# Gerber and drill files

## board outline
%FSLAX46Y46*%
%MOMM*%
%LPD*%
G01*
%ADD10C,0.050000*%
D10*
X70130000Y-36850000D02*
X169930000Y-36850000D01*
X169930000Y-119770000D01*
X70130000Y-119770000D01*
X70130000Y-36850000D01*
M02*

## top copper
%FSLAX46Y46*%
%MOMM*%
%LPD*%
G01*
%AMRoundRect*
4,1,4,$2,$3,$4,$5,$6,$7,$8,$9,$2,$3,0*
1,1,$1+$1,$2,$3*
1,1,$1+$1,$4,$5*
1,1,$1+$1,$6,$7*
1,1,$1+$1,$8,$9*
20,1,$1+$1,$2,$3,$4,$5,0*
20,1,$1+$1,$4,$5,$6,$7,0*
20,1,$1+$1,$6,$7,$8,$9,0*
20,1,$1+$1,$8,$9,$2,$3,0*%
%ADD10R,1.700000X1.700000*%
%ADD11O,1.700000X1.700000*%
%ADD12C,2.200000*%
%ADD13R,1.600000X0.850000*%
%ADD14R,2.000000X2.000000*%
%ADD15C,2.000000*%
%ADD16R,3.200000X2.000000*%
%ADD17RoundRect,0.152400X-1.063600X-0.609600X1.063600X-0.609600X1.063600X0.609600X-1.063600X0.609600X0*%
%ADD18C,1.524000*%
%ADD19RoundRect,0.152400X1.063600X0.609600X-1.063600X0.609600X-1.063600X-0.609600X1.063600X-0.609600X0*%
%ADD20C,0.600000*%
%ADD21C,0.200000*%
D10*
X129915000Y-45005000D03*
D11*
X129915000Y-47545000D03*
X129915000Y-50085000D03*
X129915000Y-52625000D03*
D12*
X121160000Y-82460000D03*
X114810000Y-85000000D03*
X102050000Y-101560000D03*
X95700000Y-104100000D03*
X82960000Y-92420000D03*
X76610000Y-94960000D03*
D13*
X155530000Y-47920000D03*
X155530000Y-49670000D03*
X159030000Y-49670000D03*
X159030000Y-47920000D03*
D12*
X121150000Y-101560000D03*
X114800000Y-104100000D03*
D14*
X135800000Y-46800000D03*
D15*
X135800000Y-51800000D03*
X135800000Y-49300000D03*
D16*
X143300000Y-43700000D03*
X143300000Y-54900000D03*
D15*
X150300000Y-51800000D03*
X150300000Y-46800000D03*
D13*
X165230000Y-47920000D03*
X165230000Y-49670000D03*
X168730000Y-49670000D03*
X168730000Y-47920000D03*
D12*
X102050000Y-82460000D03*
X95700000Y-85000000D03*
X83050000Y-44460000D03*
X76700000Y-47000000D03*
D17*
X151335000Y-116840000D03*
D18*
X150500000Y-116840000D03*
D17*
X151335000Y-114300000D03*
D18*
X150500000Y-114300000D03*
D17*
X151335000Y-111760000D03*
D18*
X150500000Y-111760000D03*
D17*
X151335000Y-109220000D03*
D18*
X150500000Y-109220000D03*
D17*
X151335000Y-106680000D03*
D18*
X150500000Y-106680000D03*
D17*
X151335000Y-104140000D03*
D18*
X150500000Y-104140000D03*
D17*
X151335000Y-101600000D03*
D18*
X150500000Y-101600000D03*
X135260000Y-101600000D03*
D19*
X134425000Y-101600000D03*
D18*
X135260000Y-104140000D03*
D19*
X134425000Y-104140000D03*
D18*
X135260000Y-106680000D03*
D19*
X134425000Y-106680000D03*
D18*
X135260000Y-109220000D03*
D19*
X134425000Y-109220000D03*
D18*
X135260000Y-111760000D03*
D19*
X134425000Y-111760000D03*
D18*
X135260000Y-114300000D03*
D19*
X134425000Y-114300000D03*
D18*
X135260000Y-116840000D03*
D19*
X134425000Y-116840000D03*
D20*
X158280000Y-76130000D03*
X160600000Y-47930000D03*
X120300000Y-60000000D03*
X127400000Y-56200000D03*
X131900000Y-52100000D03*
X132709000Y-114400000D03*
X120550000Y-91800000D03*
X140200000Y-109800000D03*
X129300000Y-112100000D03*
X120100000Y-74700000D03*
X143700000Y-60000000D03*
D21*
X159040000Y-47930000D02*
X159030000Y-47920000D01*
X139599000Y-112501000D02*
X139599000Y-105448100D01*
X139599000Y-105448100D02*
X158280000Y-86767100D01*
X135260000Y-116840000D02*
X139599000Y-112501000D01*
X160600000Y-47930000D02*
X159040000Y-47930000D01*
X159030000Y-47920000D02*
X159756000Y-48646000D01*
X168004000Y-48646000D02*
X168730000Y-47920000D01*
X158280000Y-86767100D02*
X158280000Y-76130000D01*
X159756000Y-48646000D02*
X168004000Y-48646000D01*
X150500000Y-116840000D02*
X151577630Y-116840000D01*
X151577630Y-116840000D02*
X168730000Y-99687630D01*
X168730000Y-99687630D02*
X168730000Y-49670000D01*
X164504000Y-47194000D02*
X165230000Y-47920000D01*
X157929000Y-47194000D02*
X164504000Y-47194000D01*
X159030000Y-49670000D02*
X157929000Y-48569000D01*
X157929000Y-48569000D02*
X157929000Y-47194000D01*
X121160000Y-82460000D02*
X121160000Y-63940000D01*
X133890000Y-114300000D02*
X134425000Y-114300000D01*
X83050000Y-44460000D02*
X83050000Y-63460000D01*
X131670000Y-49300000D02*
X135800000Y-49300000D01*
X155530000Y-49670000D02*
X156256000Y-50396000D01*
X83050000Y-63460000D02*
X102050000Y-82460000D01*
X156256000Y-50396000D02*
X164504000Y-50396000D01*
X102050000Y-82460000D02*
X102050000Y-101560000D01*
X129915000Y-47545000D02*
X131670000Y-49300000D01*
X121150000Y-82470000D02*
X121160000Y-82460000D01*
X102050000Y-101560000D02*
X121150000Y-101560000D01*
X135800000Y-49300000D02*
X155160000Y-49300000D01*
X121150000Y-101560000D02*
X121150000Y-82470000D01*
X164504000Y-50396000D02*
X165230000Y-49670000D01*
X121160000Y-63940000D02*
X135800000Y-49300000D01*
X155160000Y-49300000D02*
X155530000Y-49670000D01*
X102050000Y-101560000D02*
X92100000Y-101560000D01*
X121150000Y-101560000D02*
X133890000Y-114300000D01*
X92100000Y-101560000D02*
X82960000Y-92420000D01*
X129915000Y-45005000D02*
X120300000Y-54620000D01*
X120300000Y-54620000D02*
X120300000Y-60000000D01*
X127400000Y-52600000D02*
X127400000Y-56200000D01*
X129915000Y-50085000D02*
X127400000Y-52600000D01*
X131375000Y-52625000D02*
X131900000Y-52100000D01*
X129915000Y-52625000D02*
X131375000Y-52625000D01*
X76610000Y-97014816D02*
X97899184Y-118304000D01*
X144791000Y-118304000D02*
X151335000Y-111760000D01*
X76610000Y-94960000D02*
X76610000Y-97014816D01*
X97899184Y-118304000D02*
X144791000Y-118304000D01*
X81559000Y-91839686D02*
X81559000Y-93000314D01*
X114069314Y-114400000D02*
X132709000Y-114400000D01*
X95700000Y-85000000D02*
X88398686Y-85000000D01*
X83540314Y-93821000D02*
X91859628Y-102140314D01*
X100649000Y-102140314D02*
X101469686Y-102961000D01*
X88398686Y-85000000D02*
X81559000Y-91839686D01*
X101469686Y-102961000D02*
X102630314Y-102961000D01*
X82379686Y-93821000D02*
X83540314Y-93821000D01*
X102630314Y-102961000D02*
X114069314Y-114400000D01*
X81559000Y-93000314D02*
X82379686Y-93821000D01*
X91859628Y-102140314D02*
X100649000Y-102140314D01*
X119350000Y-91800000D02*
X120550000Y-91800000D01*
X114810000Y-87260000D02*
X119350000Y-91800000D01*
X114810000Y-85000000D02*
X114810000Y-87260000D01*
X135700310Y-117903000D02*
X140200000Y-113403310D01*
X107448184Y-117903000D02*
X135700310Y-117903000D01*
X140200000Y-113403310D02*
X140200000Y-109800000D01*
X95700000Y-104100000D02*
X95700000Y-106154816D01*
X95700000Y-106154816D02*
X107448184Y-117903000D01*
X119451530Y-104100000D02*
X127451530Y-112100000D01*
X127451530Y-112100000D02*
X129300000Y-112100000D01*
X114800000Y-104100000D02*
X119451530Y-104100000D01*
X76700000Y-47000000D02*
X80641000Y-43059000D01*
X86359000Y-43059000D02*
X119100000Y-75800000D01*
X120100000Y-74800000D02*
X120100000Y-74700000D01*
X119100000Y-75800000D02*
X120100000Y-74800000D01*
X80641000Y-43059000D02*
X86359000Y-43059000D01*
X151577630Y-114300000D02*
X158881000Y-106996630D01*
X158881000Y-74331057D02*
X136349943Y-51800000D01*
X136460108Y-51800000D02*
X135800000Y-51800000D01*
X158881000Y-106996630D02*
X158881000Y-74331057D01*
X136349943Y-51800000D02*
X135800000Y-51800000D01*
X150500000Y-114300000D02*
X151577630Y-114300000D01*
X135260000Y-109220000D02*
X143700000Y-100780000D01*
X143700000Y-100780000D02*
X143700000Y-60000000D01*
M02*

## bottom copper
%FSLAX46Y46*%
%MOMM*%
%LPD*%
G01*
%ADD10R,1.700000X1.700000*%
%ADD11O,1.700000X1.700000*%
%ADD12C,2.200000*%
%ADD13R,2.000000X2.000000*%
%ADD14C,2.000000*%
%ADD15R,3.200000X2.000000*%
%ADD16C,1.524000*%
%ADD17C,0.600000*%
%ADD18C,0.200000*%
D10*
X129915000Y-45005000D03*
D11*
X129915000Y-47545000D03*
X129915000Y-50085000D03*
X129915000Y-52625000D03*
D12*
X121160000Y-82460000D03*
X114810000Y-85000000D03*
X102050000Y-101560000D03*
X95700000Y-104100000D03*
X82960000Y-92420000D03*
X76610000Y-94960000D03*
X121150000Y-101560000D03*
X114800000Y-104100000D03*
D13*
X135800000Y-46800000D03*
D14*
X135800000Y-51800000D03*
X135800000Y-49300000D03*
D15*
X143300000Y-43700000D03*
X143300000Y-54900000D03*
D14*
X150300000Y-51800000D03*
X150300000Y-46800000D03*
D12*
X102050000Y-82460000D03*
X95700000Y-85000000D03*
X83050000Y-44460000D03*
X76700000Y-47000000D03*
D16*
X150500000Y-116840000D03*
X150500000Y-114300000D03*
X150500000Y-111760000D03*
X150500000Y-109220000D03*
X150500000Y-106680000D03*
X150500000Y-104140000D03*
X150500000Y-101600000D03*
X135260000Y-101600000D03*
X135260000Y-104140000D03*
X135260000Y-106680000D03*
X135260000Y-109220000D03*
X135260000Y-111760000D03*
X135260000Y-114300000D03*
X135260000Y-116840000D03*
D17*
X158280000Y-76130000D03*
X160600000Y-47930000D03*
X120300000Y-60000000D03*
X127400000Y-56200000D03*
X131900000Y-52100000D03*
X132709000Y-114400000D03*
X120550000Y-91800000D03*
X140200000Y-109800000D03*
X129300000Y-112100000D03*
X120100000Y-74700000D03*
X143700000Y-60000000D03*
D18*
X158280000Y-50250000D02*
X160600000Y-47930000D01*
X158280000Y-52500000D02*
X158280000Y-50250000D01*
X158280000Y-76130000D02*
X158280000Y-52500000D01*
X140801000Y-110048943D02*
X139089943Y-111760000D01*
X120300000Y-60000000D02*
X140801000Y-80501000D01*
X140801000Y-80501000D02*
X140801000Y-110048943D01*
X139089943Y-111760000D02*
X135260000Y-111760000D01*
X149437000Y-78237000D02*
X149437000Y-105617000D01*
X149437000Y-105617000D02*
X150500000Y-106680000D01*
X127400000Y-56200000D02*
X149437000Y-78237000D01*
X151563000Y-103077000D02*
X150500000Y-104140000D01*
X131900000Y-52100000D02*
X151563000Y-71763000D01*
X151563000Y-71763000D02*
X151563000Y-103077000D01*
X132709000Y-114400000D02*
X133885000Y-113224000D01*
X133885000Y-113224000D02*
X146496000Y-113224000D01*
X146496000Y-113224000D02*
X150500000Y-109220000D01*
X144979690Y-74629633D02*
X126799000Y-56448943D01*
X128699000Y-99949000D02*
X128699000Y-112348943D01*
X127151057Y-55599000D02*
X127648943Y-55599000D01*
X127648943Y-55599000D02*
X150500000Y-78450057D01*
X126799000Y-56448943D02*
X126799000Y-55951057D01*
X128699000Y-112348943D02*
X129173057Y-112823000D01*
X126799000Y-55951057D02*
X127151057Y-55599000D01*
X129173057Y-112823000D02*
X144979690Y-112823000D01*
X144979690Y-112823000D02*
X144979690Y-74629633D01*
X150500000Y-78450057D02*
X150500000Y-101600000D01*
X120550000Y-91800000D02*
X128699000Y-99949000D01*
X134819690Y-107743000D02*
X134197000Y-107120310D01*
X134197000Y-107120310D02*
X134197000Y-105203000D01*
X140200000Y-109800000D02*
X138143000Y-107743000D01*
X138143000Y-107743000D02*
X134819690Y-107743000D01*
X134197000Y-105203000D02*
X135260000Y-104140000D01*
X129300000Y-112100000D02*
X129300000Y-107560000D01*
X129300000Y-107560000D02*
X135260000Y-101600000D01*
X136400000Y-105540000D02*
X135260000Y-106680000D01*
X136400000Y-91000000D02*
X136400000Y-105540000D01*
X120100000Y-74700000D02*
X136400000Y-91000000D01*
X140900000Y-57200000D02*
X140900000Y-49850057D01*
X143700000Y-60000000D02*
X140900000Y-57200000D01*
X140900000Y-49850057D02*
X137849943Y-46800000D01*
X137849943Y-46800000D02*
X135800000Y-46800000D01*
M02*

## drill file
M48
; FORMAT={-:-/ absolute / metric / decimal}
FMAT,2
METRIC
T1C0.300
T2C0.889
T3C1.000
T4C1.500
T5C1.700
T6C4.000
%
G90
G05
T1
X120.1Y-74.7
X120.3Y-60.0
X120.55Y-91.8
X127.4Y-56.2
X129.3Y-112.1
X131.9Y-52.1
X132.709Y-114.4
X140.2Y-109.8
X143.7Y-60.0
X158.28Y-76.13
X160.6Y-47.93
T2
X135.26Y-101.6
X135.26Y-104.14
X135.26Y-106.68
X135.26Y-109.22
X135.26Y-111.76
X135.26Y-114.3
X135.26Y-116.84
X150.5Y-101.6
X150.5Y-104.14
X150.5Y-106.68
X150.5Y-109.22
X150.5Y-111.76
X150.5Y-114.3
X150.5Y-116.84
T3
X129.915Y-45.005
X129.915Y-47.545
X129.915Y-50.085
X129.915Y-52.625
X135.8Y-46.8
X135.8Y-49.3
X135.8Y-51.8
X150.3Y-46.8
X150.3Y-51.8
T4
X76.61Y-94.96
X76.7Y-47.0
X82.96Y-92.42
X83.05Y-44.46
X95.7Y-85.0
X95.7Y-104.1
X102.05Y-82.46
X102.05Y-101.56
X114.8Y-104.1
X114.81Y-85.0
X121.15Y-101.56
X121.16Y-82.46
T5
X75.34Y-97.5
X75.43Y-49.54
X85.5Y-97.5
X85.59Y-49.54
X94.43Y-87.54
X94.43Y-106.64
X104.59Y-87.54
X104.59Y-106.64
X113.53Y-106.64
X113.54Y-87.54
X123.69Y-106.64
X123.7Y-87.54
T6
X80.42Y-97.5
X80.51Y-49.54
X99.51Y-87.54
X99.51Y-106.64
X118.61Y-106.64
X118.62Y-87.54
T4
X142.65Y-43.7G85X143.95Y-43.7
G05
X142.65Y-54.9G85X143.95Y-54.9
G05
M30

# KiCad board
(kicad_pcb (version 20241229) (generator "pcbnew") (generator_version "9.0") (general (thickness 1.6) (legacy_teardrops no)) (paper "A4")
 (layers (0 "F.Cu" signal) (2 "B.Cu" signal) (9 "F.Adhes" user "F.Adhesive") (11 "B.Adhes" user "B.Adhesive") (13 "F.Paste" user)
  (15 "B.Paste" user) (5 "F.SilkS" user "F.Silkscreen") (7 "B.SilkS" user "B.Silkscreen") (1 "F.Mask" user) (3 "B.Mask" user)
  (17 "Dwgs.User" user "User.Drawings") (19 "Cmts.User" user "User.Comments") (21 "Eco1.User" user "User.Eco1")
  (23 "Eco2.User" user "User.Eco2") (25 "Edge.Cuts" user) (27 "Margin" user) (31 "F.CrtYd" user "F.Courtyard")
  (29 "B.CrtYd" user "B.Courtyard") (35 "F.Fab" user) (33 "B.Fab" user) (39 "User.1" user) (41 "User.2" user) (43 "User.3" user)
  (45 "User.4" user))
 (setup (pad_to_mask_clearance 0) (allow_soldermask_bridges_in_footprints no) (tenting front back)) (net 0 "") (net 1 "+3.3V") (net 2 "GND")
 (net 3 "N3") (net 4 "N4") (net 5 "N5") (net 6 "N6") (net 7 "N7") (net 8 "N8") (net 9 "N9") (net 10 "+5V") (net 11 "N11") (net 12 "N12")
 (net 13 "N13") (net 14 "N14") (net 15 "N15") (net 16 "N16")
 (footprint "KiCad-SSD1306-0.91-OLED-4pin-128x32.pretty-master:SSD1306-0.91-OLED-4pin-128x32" (layer "F.Cu") (at 93.415 42.815)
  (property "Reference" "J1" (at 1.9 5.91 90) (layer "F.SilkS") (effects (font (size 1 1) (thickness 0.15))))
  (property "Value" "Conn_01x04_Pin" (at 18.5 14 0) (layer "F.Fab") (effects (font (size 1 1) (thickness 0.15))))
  (pad "1" thru_hole rect (at 36.5 2.19) (size 1.7 1.7) (drill 1) (layers "*.Cu" "*.Mask") (remove_unused_layers no) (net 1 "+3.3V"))
  (pad "2" thru_hole oval (at 36.5 4.73) (size 1.7 1.7) (drill 1) (layers "*.Cu" "*.Mask") (remove_unused_layers no) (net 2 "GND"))
  (pad "3" thru_hole oval (at 36.5 7.27) (size 1.7 1.7) (drill 1) (layers "*.Cu" "*.Mask") (remove_unused_layers no) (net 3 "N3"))
  (pad "4" thru_hole oval (at 36.5 9.81) (size 1.7 1.7) (drill 1) (layers "*.Cu" "*.Mask") (remove_unused_layers no) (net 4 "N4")))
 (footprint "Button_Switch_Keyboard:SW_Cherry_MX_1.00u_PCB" (layer "F.Cu") (at 121.16 82.46)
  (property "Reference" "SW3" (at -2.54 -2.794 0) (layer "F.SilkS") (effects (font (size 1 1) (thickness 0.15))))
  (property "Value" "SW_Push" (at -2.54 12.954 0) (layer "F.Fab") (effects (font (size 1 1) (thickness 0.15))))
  (pad "" np_thru_hole circle (at -7.62 5.08) (size 1.7 1.7) (drill 1.7) (layers "*.Cu" "*.Mask"))
  (pad "" np_thru_hole circle (at -2.54 5.08) (size 4 4) (drill 4) (layers "*.Cu" "*.Mask"))
  (pad "" np_thru_hole circle (at 2.54 5.08) (size 1.7 1.7) (drill 1.7) (layers "*.Cu" "*.Mask"))
  (pad "1" thru_hole circle (at 0 0) (size 2.2 2.2) (drill 1.5) (layers "*.Cu" "*.Mask") (remove_unused_layers no) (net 2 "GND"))
  (pad "2" thru_hole circle (at -6.35 2.54) (size 2.2 2.2) (drill 1.5) (layers "*.Cu" "*.Mask") (remove_unused_layers no) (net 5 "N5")))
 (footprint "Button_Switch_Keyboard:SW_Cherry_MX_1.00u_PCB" (layer "F.Cu") (at 102.05 101.56)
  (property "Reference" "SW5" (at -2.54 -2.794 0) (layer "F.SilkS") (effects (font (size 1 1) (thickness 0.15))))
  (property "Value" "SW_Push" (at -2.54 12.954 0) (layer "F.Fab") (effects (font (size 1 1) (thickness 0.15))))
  (pad "" np_thru_hole circle (at -7.62 5.08) (size 1.7 1.7) (drill 1.7) (layers "*.Cu" "*.Mask"))
  (pad "" np_thru_hole circle (at -2.54 5.08) (size 4 4) (drill 4) (layers "*.Cu" "*.Mask"))
  (pad "" np_thru_hole circle (at 2.54 5.08) (size 1.7 1.7) (drill 1.7) (layers "*.Cu" "*.Mask"))
  (pad "1" thru_hole circle (at 0 0) (size 2.2 2.2) (drill 1.5) (layers "*.Cu" "*.Mask") (remove_unused_layers no) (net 2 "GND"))
  (pad "2" thru_hole circle (at -6.35 2.54) (size 2.2 2.2) (drill 1.5) (layers "*.Cu" "*.Mask") (remove_unused_layers no) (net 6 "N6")))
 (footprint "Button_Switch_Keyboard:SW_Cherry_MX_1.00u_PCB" (layer "F.Cu") (at 82.96 92.42)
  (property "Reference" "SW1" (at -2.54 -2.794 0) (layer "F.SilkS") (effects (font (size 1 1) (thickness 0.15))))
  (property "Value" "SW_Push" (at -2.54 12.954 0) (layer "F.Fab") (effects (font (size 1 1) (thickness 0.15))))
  (pad "" np_thru_hole circle (at -7.62 5.08) (size 1.7 1.7) (drill 1.7) (layers "*.Cu" "*.Mask"))
  (pad "" np_thru_hole circle (at -2.54 5.08) (size 4 4) (drill 4) (layers "*.Cu" "*.Mask"))
  (pad "" np_thru_hole circle (at 2.54 5.08) (size 1.7 1.7) (drill 1.7) (layers "*.Cu" "*.Mask"))
  (pad "1" thru_hole circle (at 0 0) (size 2.2 2.2) (drill 1.5) (layers "*.Cu" "*.Mask") (remove_unused_layers no) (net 2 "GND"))
  (pad "2" thru_hole circle (at -6.35 2.54) (size 2.2 2.2) (drill 1.5) (layers "*.Cu" "*.Mask") (remove_unused_layers no) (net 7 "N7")))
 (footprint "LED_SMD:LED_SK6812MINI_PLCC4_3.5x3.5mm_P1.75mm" (layer "F.Cu") (at 157.28 48.795)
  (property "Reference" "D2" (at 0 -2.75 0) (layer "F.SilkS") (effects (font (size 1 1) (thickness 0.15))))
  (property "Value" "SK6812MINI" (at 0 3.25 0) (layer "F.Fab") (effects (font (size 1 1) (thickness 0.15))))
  (pad "1" smd rect (at -1.75 -0.875) (size 1.6 0.85) (layers "F.Cu" "F.Mask" "F.Paste") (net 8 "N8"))
  (pad "2" smd rect (at -1.75 0.875) (size 1.6 0.85) (layers "F.Cu" "F.Mask" "F.Paste") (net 2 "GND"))
  (pad "3" smd rect (at 1.75 0.875) (size 1.6 0.85) (layers "F.Cu" "F.Mask" "F.Paste") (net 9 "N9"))
  (pad "4" smd rect (at 1.75 -0.875) (size 1.6 0.85) (layers "F.Cu" "F.Mask" "F.Paste") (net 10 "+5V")))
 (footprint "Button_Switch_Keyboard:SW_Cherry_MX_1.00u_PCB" (layer "F.Cu") (at 121.15 101.56)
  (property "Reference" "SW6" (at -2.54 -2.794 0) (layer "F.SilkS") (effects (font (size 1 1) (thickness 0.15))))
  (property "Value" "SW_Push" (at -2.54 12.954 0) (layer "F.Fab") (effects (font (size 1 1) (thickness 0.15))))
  (pad "" np_thru_hole circle (at -7.62 5.08) (size 1.7 1.7) (drill 1.7) (layers "*.Cu" "*.Mask"))
  (pad "" np_thru_hole circle (at -2.54 5.08) (size 4 4) (drill 4) (layers "*.Cu" "*.Mask"))
  (pad "" np_thru_hole circle (at 2.54 5.08) (size 1.7 1.7) (drill 1.7) (layers "*.Cu" "*.Mask"))
  (pad "1" thru_hole circle (at 0 0) (size 2.2 2.2) (drill 1.5) (layers "*.Cu" "*.Mask") (remove_unused_layers no) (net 2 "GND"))
  (pad "2" thru_hole circle (at -6.35 2.54) (size 2.2 2.2) (drill 1.5) (layers "*.Cu" "*.Mask") (remove_unused_layers no) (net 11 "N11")))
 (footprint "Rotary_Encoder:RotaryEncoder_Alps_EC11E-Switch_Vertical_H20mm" (layer "F.Cu") (at 135.8 46.8)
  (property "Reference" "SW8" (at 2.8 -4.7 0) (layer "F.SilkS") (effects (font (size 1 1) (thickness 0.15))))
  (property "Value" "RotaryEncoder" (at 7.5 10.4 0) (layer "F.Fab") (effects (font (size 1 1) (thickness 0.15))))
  (pad "A" thru_hole rect (at 0 0) (size 2 2) (drill 1) (layers "*.Cu" "*.Mask") (remove_unused_layers no) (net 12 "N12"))
  (pad "B" thru_hole circle (at 0 5) (size 2 2) (drill 1) (layers "*.Cu" "*.Mask") (remove_unused_layers no) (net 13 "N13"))
  (pad "C" thru_hole circle (at 0 2.5) (size 2 2) (drill 1) (layers "*.Cu" "*.Mask") (remove_unused_layers no) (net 2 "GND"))
  (pad "MP" thru_hole rect (at 7.5 -3.1) (size 3.2 2) (drill oval 2.8 1.5) (layers "*.Cu" "*.Mask") (remove_unused_layers no))
  (pad "MP" thru_hole rect (at 7.5 8.1) (size 3.2 2) (drill oval 2.8 1.5) (layers "*.Cu" "*.Mask") (remove_unused_layers no))
  (pad "S1" thru_hole circle (at 14.5 5) (size 2 2) (drill 1) (layers "*.Cu" "*.Mask") (remove_unused_layers no))
  (pad "S2" thru_hole circle (at 14.5 0) (size 2 2) (drill 1) (layers "*.Cu" "*.Mask") (remove_unused_layers no)))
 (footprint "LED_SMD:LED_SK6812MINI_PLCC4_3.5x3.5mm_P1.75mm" (layer "F.Cu") (at 166.98 48.795)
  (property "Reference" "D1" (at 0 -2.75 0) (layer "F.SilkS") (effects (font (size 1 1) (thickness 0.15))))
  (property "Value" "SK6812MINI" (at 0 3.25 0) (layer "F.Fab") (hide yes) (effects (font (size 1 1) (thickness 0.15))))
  (pad "1" smd rect (at -1.75 -0.875) (size 1.6 0.85) (layers "F.Cu" "F.Mask" "F.Paste") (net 9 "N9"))
  (pad "2" smd rect (at -1.75 0.875) (size 1.6 0.85) (layers "F.Cu" "F.Mask" "F.Paste") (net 2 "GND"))
  (pad "3" smd rect (at 1.75 0.875) (size 1.6 0.85) (layers "F.Cu" "F.Mask" "F.Paste") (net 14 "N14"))
  (pad "4" smd rect (at 1.75 -0.875) (size 1.6 0.85) (layers "F.Cu" "F.Mask" "F.Paste") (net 10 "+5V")))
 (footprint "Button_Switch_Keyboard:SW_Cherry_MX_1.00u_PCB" (layer "F.Cu") (at 102.05 82.46)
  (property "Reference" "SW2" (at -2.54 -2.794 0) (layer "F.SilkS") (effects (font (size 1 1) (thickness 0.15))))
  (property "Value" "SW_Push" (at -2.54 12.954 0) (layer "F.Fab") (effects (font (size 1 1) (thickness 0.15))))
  (pad "" np_thru_hole circle (at -7.62 5.08) (size 1.7 1.7) (drill 1.7) (layers "*.Cu" "*.Mask"))
  (pad "" np_thru_hole circle (at -2.54 5.08) (size 4 4) (drill 4) (layers "*.Cu" "*.Mask"))
  (pad "" np_thru_hole circle (at 2.54 5.08) (size 1.7 1.7) (drill 1.7) (layers "*.Cu" "*.Mask"))
  (pad "1" thru_hole circle (at 0 0) (size 2.2 2.2) (drill 1.5) (layers "*.Cu" "*.Mask") (remove_unused_layers no) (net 2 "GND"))
  (pad "2" thru_hole circle (at -6.35 2.54) (size 2.2 2.2) (drill 1.5) (layers "*.Cu" "*.Mask") (remove_unused_layers no) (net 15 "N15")))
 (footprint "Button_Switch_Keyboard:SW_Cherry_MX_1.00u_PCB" (layer "F.Cu") (at 83.05 44.46)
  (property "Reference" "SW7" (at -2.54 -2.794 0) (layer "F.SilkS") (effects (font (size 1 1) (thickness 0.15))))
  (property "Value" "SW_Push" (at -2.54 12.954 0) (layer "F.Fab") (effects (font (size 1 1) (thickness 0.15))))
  (pad "" np_thru_hole circle (at -7.62 5.08) (size 1.7 1.7) (drill 1.7) (layers "*.Cu" "*.Mask"))
  (pad "" np_thru_hole circle (at -2.54 5.08) (size 4 4) (drill 4) (layers "*.Cu" "*.Mask"))
  (pad "" np_thru_hole circle (at 2.54 5.08) (size 1.7 1.7) (drill 1.7) (layers "*.Cu" "*.Mask"))
  (pad "1" thru_hole circle (at 0 0) (size 2.2 2.2) (drill 1.5) (layers "*.Cu" "*.Mask") (remove_unused_layers no) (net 2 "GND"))
  (pad "2" thru_hole circle (at -6.35 2.54) (size 2.2 2.2) (drill 1.5) (layers "*.Cu" "*.Mask") (remove_unused_layers no) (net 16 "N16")))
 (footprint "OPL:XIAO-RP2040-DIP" (layer "F.Cu") (at 142.88 109.22 180)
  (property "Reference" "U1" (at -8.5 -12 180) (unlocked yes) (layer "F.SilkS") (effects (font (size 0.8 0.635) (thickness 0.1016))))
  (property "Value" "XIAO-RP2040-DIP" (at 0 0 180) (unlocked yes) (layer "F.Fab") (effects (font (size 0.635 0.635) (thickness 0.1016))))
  (pad "1" smd roundrect (at -8.455 -7.62) (size 2.432 1.524) (layers "F.Cu" "F.Mask") (roundrect_rratio 0.1) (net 14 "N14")
   (thermal_bridge_angle 45))
  (pad "1" thru_hole circle (at -7.62 -7.62) (size 1.524 1.524) (drill 0.889) (layers "*.Cu" "*.Mask") (remove_unused_layers no)
   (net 14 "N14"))
  (pad "2" smd roundrect (at -8.455 -5.08) (size 2.432 1.524) (layers "F.Cu" "F.Mask") (roundrect_rratio 0.1) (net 13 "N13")
   (thermal_bridge_angle 45))
  (pad "2" thru_hole circle (at -7.62 -5.08) (size 1.524 1.524) (drill 0.889) (layers "*.Cu" "*.Mask") (remove_unused_layers no)
   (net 13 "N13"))
  (pad "3" smd roundrect (at -8.455 -2.54) (size 2.432 1.524) (layers "F.Cu" "F.Mask") (roundrect_rratio 0.1) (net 7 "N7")
   (thermal_bridge_angle 45))
  (pad "3" thru_hole circle (at -7.62 -2.54) (size 1.524 1.524) (drill 0.889) (layers "*.Cu" "*.Mask") (remove_unused_layers no)
   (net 7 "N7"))
  (pad "4" smd roundrect (at -8.455 0) (size 2.432 1.524) (layers "F.Cu" "F.Mask") (roundrect_rratio 0.1) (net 15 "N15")
   (thermal_bridge_angle 45))
  (pad "4" thru_hole circle (at -7.62 0) (size 1.524 1.524) (drill 0.889) (layers "*.Cu" "*.Mask") (remove_unused_layers no) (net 15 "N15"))
  (pad "5" smd roundrect (at -8.455 2.54) (size 2.432 1.524) (layers "F.Cu" "F.Mask") (roundrect_rratio 0.1) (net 3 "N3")
   (thermal_bridge_angle 45))
  (pad "5" thru_hole circle (at -7.62 2.54) (size 1.524 1.524) (drill 0.889) (layers "*.Cu" "*.Mask") (remove_unused_layers no) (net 3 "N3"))
  (pad "6" smd roundrect (at -8.455 5.08) (size 2.432 1.524) (layers "F.Cu" "F.Mask") (roundrect_rratio 0.1) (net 4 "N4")
   (thermal_bridge_angle 45))
  (pad "6" thru_hole circle (at -7.62 5.08) (size 1.524 1.524) (drill 0.889) (layers "*.Cu" "*.Mask") (remove_unused_layers no) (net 4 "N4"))
  (pad "7" smd roundrect (at -8.455 7.62) (size 2.432 1.524) (layers "F.Cu" "F.Mask") (roundrect_rratio 0.1) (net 5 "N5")
   (thermal_bridge_angle 45))
  (pad "7" thru_hole circle (at -7.62 7.62) (size 1.524 1.524) (drill 0.889) (layers "*.Cu" "*.Mask") (remove_unused_layers no) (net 5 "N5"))
  (pad "8" thru_hole circle (at 7.62 7.62 180) (size 1.524 1.524) (drill 0.889) (layers "*.Cu" "*.Mask") (remove_unused_layers no)
   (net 11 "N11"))
  (pad "8" smd roundrect (at 8.455 7.62 180) (size 2.432 1.524) (layers "F.Cu" "F.Mask") (roundrect_rratio 0.1) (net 11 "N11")
   (thermal_bridge_angle 45))
  (pad "9" thru_hole circle (at 7.62 5.08 180) (size 1.524 1.524) (drill 0.889) (layers "*.Cu" "*.Mask") (remove_unused_layers no)
   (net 6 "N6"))
  (pad "9" smd roundrect (at 8.455 5.08 180) (size 2.432 1.524) (layers "F.Cu" "F.Mask") (roundrect_rratio 0.1) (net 6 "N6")
   (thermal_bridge_angle 45))
  (pad "10" thru_hole circle (at 7.62 2.54 180) (size 1.524 1.524) (drill 0.889) (layers "*.Cu" "*.Mask") (remove_unused_layers no)
   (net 16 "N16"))
  (pad "10" smd roundrect (at 8.455 2.54 180) (size 2.432 1.524) (layers "F.Cu" "F.Mask") (roundrect_rratio 0.1) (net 16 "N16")
   (thermal_bridge_angle 45))
  (pad "11" thru_hole circle (at 7.62 0 180) (size 1.524 1.524) (drill 0.889) (layers "*.Cu" "*.Mask") (remove_unused_layers no)
   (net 12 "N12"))
  (pad "11" smd roundrect (at 8.455 0 180) (size 2.432 1.524) (layers "F.Cu" "F.Mask") (roundrect_rratio 0.1) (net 12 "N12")
   (thermal_bridge_angle 45))
  (pad "12" thru_hole circle (at 7.62 -2.54 180) (size 1.524 1.524) (drill 0.889) (layers "*.Cu" "*.Mask") (remove_unused_layers no)
   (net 1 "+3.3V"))
  (pad "12" smd roundrect (at 8.455 -2.54 180) (size 2.432 1.524) (layers "F.Cu" "F.Mask") (roundrect_rratio 0.1) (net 1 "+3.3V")
   (thermal_bridge_angle 45))
  (pad "13" thru_hole circle (at 7.62 -5.08 180) (size 1.524 1.524) (drill 0.889) (layers "*.Cu" "*.Mask") (remove_unused_layers no)
   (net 2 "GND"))
  (pad "13" smd roundrect (at 8.455 -5.08 180) (size 2.432 1.524) (layers "F.Cu" "F.Mask") (roundrect_rratio 0.1) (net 2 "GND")
   (thermal_bridge_angle 45))
  (pad "14" thru_hole circle (at 7.62 -7.62 180) (size 1.524 1.524) (drill 0.889) (layers "*.Cu" "*.Mask") (remove_unused_layers no)
   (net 10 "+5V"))
  (pad "14" smd roundrect (at 8.455 -7.62 180) (size 2.432 1.524) (layers "F.Cu" "F.Mask") (roundrect_rratio 0.1) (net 10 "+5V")
   (thermal_bridge_angle 45)))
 (gr_rect (start 70.13 36.85) (end 169.93 119.77) (stroke (width 0.05) (type default)) (fill no) (layer "Edge.Cuts"))
 (segment (start 159.04 47.93) (end 159.03 47.92) (width 0.2) (layer "F.Cu") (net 10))
 (segment (start 139.599 112.501) (end 139.599 105.4481) (width 0.2) (layer "F.Cu") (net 10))
 (segment (start 139.599 105.4481) (end 158.28 86.7671) (width 0.2) (layer "F.Cu") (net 10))
 (segment (start 135.26 116.84) (end 139.599 112.501) (width 0.2) (layer "F.Cu") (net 10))
 (segment (start 160.6 47.93) (end 159.04 47.93) (width 0.2) (layer "F.Cu") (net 10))
 (segment (start 159.03 47.92) (end 159.756 48.646) (width 0.2) (layer "F.Cu") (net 10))
 (segment (start 168.004 48.646) (end 168.73 47.92) (width 0.2) (layer "F.Cu") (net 10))
 (segment (start 158.28 86.7671) (end 158.28 76.13) (width 0.2) (layer "F.Cu") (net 10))
 (segment (start 159.756 48.646) (end 168.004 48.646) (width 0.2) (layer "F.Cu") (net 10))
 (via (at 158.28 76.13) (size 0.6) (drill 0.3) (layers "F.Cu" "B.Cu") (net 10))
 (via (at 160.6 47.93) (size 0.6) (drill 0.3) (layers "F.Cu" "B.Cu") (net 10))
 (segment (start 158.28 50.25) (end 160.6 47.93) (width 0.2) (layer "B.Cu") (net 10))
 (segment (start 158.28 52.5) (end 158.28 50.25) (width 0.2) (layer "B.Cu") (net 10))
 (segment (start 158.28 76.13) (end 158.28 52.5) (width 0.2) (layer "B.Cu") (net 10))
 (segment (start 150.5 116.84) (end 151.57763 116.84) (width 0.2) (layer "F.Cu") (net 14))
 (segment (start 151.57763 116.84) (end 168.73 99.68763) (width 0.2) (layer "F.Cu") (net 14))
 (segment (start 168.73 99.68763) (end 168.73 49.67) (width 0.2) (layer "F.Cu") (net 14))
 (segment (start 164.504 47.194) (end 165.23 47.92) (width 0.2) (layer "F.Cu") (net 9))
 (segment (start 157.929 47.194) (end 164.504 47.194) (width 0.2) (layer "F.Cu") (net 9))
 (segment (start 159.03 49.67) (end 157.929 48.569) (width 0.2) (layer "F.Cu") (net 9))
 (segment (start 157.929 48.569) (end 157.929 47.194) (width 0.2) (layer "F.Cu") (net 9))
 (segment (start 121.16 82.46) (end 121.16 63.94) (width 0.2) (layer "F.Cu") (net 2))
 (segment (start 133.89 114.3) (end 134.425 114.3) (width 0.2) (layer "F.Cu") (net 2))
 (segment (start 83.05 44.46) (end 83.05 63.46) (width 0.2) (layer "F.Cu") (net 2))
 (segment (start 131.67 49.3) (end 135.8 49.3) (width 0.2) (layer "F.Cu") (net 2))
 (segment (start 155.53 49.67) (end 156.256 50.396) (width 0.2) (layer "F.Cu") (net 2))
 (segment (start 83.05 63.46) (end 102.05 82.46) (width 0.2) (layer "F.Cu") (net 2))
 (segment (start 156.256 50.396) (end 164.504 50.396) (width 0.2) (layer "F.Cu") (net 2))
 (segment (start 102.05 82.46) (end 102.05 101.56) (width 0.2) (layer "F.Cu") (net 2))
 (segment (start 129.915 47.545) (end 131.67 49.3) (width 0.2) (layer "F.Cu") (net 2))
 (segment (start 121.15 82.47) (end 121.16 82.46) (width 0.2) (layer "F.Cu") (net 2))
 (segment (start 102.05 101.56) (end 121.15 101.56) (width 0.2) (layer "F.Cu") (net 2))
 (segment (start 135.8 49.3) (end 155.16 49.3) (width 0.2) (layer "F.Cu") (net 2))
 (segment (start 121.15 101.56) (end 121.15 82.47) (width 0.2) (layer "F.Cu") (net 2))
 (segment (start 164.504 50.396) (end 165.23 49.67) (width 0.2) (layer "F.Cu") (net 2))
 (segment (start 121.16 63.94) (end 135.8 49.3) (width 0.2) (layer "F.Cu") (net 2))
 (segment (start 155.16 49.3) (end 155.53 49.67) (width 0.2) (layer "F.Cu") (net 2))
 (segment (start 102.05 101.56) (end 92.1 101.56) (width 0.2) (layer "F.Cu") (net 2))
 (segment (start 121.15 101.56) (end 133.89 114.3) (width 0.2) (layer "F.Cu") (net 2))
 (segment (start 92.1 101.56) (end 82.96 92.42) (width 0.2) (layer "F.Cu") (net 2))
 (segment (start 129.915 45.005) (end 120.3 54.62) (width 0.2) (layer "F.Cu") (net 1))
 (segment (start 120.3 54.62) (end 120.3 60) (width 0.2) (layer "F.Cu") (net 1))
 (via (at 120.3 60) (size 0.6) (drill 0.3) (layers "F.Cu" "B.Cu") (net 1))
 (segment (start 140.801 110.048943) (end 139.089943 111.76) (width 0.2) (layer "B.Cu") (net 1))
 (segment (start 120.3 60) (end 140.801 80.501) (width 0.2) (layer "B.Cu") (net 1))
 (segment (start 140.801 80.501) (end 140.801 110.048943) (width 0.2) (layer "B.Cu") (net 1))
 (segment (start 139.089943 111.76) (end 135.26 111.76) (width 0.2) (layer "B.Cu") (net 1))
 (segment (start 127.4 52.6) (end 127.4 56.2) (width 0.2) (layer "F.Cu") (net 3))
 (segment (start 129.915 50.085) (end 127.4 52.6) (width 0.2) (layer "F.Cu") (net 3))
 (via (at 127.4 56.2) (size 0.6) (drill 0.3) (layers "F.Cu" "B.Cu") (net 3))
 (segment (start 149.437 78.237) (end 149.437 105.617) (width 0.2) (layer "B.Cu") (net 3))
 (segment (start 149.437 105.617) (end 150.5 106.68) (width 0.2) (layer "B.Cu") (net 3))
 (segment (start 127.4 56.2) (end 149.437 78.237) (width 0.2) (layer "B.Cu") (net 3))
 (segment (start 131.375 52.625) (end 131.9 52.1) (width 0.2) (layer "F.Cu") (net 4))
 (segment (start 129.915 52.625) (end 131.375 52.625) (width 0.2) (layer "F.Cu") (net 4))
 (via (at 131.9 52.1) (size 0.6) (drill 0.3) (layers "F.Cu" "B.Cu") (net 4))
 (segment (start 151.563 103.077) (end 150.5 104.14) (width 0.2) (layer "B.Cu") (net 4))
 (segment (start 131.9 52.1) (end 151.563 71.763) (width 0.2) (layer "B.Cu") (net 4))
 (segment (start 151.563 71.763) (end 151.563 103.077) (width 0.2) (layer "B.Cu") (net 4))
 (segment (start 76.61 97.014816) (end 97.899184 118.304) (width 0.2) (layer "F.Cu") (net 7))
 (segment (start 144.791 118.304) (end 151.335 111.76) (width 0.2) (layer "F.Cu") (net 7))
 (segment (start 76.61 94.96) (end 76.61 97.014816) (width 0.2) (layer "F.Cu") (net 7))
 (segment (start 97.899184 118.304) (end 144.791 118.304) (width 0.2) (layer "F.Cu") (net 7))
 (segment (start 81.559 91.839686) (end 81.559 93.000314) (width 0.2) (layer "F.Cu") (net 15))
 (segment (start 114.069314 114.4) (end 132.709 114.4) (width 0.2) (layer "F.Cu") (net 15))
 (segment (start 95.7 85) (end 88.398686 85) (width 0.2) (layer "F.Cu") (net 15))
 (segment (start 83.540314 93.821) (end 91.859628 102.140314) (width 0.2) (layer "F.Cu") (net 15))
 (segment (start 100.649 102.140314) (end 101.469686 102.961) (width 0.2) (layer "F.Cu") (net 15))
 (segment (start 88.398686 85) (end 81.559 91.839686) (width 0.2) (layer "F.Cu") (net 15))
 (segment (start 101.469686 102.961) (end 102.630314 102.961) (width 0.2) (layer "F.Cu") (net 15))
 (segment (start 82.379686 93.821) (end 83.540314 93.821) (width 0.2) (layer "F.Cu") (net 15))
 (segment (start 102.630314 102.961) (end 114.069314 114.4) (width 0.2) (layer "F.Cu") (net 15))
 (segment (start 81.559 93.000314) (end 82.379686 93.821) (width 0.2) (layer "F.Cu") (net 15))
 (segment (start 91.859628 102.140314) (end 100.649 102.140314) (width 0.2) (layer "F.Cu") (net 15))
 (via (at 132.709 114.4) (size 0.6) (drill 0.3) (layers "F.Cu" "B.Cu") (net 15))
 (segment (start 132.709 114.4) (end 133.885 113.224) (width 0.2) (layer "B.Cu") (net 15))
 (segment (start 133.885 113.224) (end 146.496 113.224) (width 0.2) (layer "B.Cu") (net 15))
 (segment (start 146.496 113.224) (end 150.5 109.22) (width 0.2) (layer "B.Cu") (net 15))
 (segment (start 119.35 91.8) (end 120.55 91.8) (width 0.2) (layer "F.Cu") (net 5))
 (segment (start 114.81 87.26) (end 119.35 91.8) (width 0.2) (layer "F.Cu") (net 5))
 (segment (start 114.81 85) (end 114.81 87.26) (width 0.2) (layer "F.Cu") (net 5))
 (via (at 120.55 91.8) (size 0.6) (drill 0.3) (layers "F.Cu" "B.Cu") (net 5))
 (segment (start 144.97969 74.629633) (end 126.799 56.448943) (width 0.2) (layer "B.Cu") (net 5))
 (segment (start 128.699 99.949) (end 128.699 112.348943) (width 0.2) (layer "B.Cu") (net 5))
 (segment (start 127.151057 55.599) (end 127.648943 55.599) (width 0.2) (layer "B.Cu") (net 5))
 (segment (start 127.648943 55.599) (end 150.5 78.450057) (width 0.2) (layer "B.Cu") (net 5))
 (segment (start 126.799 56.448943) (end 126.799 55.951057) (width 0.2) (layer "B.Cu") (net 5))
 (segment (start 128.699 112.348943) (end 129.173057 112.823) (width 0.2) (layer "B.Cu") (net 5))
 (segment (start 126.799 55.951057) (end 127.151057 55.599) (width 0.2) (layer "B.Cu") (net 5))
 (segment (start 129.173057 112.823) (end 144.97969 112.823) (width 0.2) (layer "B.Cu") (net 5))
 (segment (start 144.97969 112.823) (end 144.97969 74.629633) (width 0.2) (layer "B.Cu") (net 5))
 (segment (start 150.5 78.450057) (end 150.5 101.6) (width 0.2) (layer "B.Cu") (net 5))
 (segment (start 120.55 91.8) (end 128.699 99.949) (width 0.2) (layer "B.Cu") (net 5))
 (segment (start 135.70031 117.903) (end 140.2 113.40331) (width 0.2) (layer "F.Cu") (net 6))
 (segment (start 107.448184 117.903) (end 135.70031 117.903) (width 0.2) (layer "F.Cu") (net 6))
 (segment (start 140.2 113.40331) (end 140.2 109.8) (width 0.2) (layer "F.Cu") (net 6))
 (segment (start 95.7 104.1) (end 95.7 106.154816) (width 0.2) (layer "F.Cu") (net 6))
 (segment (start 95.7 106.154816) (end 107.448184 117.903) (width 0.2) (layer "F.Cu") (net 6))
 (via (at 140.2 109.8) (size 0.6) (drill 0.3) (layers "F.Cu" "B.Cu") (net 6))
 (segment (start 134.81969 107.743) (end 134.197 107.12031) (width 0.2) (layer "B.Cu") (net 6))
 (segment (start 134.197 107.12031) (end 134.197 105.203) (width 0.2) (layer "B.Cu") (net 6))
 (segment (start 140.2 109.8) (end 138.143 107.743) (width 0.2) (layer "B.Cu") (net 6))
 (segment (start 138.143 107.743) (end 134.81969 107.743) (width 0.2) (layer "B.Cu") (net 6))
 (segment (start 134.197 105.203) (end 135.26 104.14) (width 0.2) (layer "B.Cu") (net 6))
 (segment (start 119.45153 104.1) (end 127.45153 112.1) (width 0.2) (layer "F.Cu") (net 11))
 (segment (start 127.45153 112.1) (end 129.3 112.1) (width 0.2) (layer "F.Cu") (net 11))
 (segment (start 114.8 104.1) (end 119.45153 104.1) (width 0.2) (layer "F.Cu") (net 11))
 (via (at 129.3 112.1) (size 0.6) (drill 0.3) (layers "F.Cu" "B.Cu") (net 11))
 (segment (start 129.3 112.1) (end 129.3 107.56) (width 0.2) (layer "B.Cu") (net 11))
 (segment (start 129.3 107.56) (end 135.26 101.6) (width 0.2) (layer "B.Cu") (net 11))
 (segment (start 76.7 47) (end 80.641 43.059) (width 0.2) (layer "F.Cu") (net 16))
 (segment (start 86.359 43.059) (end 119.1 75.8) (width 0.2) (layer "F.Cu") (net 16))
 (segment (start 120.1 74.8) (end 120.1 74.7) (width 0.2) (layer "F.Cu") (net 16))
 (segment (start 119.1 75.8) (end 120.1 74.8) (width 0.2) (layer "F.Cu") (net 16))
 (segment (start 80.641 43.059) (end 86.359 43.059) (width 0.2) (layer "F.Cu") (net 16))
 (via (at 120.1 74.7) (size 0.6) (drill 0.3) (layers "F.Cu" "B.Cu") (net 16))
 (segment (start 136.4 105.54) (end 135.26 106.68) (width 0.2) (layer "B.Cu") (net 16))
 (segment (start 136.4 91) (end 136.4 105.54) (width 0.2) (layer "B.Cu") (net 16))
 (segment (start 120.1 74.7) (end 136.4 91) (width 0.2) (layer "B.Cu") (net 16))
 (segment (start 151.57763 114.3) (end 158.881 106.99663) (width 0.2) (layer "F.Cu") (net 13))
 (segment (start 158.881 74.331057) (end 136.349943 51.8) (width 0.2) (layer "F.Cu") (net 13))
 (segment (start 136.460108 51.8) (end 135.8 51.8) (width 0.2) (layer "F.Cu") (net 13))
 (segment (start 158.881 106.99663) (end 158.881 74.331057) (width 0.2) (layer "F.Cu") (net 13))
 (segment (start 136.349943 51.8) (end 135.8 51.8) (width 0.2) (layer "F.Cu") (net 13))
 (segment (start 150.5 114.3) (end 151.57763 114.3) (width 0.2) (layer "F.Cu") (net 13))
 (segment (start 135.26 109.22) (end 143.7 100.78) (width 0.2) (layer "F.Cu") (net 12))
 (segment (start 143.7 100.78) (end 143.7 60) (width 0.2) (layer "F.Cu") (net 12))
 (via (at 143.7 60) (size 0.6) (drill 0.3) (layers "F.Cu" "B.Cu") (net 12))
 (segment (start 140.9 57.2) (end 140.9 49.850057) (width 0.2) (layer "B.Cu") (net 12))
 (segment (start 143.7 60) (end 140.9 57.2) (width 0.2) (layer "B.Cu") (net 12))
 (segment (start 140.9 49.850057) (end 137.849943 46.8) (width 0.2) (layer "B.Cu") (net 12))
 (segment (start 137.849943 46.8) (end 135.8 46.8) (width 0.2) (layer "B.Cu") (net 12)))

